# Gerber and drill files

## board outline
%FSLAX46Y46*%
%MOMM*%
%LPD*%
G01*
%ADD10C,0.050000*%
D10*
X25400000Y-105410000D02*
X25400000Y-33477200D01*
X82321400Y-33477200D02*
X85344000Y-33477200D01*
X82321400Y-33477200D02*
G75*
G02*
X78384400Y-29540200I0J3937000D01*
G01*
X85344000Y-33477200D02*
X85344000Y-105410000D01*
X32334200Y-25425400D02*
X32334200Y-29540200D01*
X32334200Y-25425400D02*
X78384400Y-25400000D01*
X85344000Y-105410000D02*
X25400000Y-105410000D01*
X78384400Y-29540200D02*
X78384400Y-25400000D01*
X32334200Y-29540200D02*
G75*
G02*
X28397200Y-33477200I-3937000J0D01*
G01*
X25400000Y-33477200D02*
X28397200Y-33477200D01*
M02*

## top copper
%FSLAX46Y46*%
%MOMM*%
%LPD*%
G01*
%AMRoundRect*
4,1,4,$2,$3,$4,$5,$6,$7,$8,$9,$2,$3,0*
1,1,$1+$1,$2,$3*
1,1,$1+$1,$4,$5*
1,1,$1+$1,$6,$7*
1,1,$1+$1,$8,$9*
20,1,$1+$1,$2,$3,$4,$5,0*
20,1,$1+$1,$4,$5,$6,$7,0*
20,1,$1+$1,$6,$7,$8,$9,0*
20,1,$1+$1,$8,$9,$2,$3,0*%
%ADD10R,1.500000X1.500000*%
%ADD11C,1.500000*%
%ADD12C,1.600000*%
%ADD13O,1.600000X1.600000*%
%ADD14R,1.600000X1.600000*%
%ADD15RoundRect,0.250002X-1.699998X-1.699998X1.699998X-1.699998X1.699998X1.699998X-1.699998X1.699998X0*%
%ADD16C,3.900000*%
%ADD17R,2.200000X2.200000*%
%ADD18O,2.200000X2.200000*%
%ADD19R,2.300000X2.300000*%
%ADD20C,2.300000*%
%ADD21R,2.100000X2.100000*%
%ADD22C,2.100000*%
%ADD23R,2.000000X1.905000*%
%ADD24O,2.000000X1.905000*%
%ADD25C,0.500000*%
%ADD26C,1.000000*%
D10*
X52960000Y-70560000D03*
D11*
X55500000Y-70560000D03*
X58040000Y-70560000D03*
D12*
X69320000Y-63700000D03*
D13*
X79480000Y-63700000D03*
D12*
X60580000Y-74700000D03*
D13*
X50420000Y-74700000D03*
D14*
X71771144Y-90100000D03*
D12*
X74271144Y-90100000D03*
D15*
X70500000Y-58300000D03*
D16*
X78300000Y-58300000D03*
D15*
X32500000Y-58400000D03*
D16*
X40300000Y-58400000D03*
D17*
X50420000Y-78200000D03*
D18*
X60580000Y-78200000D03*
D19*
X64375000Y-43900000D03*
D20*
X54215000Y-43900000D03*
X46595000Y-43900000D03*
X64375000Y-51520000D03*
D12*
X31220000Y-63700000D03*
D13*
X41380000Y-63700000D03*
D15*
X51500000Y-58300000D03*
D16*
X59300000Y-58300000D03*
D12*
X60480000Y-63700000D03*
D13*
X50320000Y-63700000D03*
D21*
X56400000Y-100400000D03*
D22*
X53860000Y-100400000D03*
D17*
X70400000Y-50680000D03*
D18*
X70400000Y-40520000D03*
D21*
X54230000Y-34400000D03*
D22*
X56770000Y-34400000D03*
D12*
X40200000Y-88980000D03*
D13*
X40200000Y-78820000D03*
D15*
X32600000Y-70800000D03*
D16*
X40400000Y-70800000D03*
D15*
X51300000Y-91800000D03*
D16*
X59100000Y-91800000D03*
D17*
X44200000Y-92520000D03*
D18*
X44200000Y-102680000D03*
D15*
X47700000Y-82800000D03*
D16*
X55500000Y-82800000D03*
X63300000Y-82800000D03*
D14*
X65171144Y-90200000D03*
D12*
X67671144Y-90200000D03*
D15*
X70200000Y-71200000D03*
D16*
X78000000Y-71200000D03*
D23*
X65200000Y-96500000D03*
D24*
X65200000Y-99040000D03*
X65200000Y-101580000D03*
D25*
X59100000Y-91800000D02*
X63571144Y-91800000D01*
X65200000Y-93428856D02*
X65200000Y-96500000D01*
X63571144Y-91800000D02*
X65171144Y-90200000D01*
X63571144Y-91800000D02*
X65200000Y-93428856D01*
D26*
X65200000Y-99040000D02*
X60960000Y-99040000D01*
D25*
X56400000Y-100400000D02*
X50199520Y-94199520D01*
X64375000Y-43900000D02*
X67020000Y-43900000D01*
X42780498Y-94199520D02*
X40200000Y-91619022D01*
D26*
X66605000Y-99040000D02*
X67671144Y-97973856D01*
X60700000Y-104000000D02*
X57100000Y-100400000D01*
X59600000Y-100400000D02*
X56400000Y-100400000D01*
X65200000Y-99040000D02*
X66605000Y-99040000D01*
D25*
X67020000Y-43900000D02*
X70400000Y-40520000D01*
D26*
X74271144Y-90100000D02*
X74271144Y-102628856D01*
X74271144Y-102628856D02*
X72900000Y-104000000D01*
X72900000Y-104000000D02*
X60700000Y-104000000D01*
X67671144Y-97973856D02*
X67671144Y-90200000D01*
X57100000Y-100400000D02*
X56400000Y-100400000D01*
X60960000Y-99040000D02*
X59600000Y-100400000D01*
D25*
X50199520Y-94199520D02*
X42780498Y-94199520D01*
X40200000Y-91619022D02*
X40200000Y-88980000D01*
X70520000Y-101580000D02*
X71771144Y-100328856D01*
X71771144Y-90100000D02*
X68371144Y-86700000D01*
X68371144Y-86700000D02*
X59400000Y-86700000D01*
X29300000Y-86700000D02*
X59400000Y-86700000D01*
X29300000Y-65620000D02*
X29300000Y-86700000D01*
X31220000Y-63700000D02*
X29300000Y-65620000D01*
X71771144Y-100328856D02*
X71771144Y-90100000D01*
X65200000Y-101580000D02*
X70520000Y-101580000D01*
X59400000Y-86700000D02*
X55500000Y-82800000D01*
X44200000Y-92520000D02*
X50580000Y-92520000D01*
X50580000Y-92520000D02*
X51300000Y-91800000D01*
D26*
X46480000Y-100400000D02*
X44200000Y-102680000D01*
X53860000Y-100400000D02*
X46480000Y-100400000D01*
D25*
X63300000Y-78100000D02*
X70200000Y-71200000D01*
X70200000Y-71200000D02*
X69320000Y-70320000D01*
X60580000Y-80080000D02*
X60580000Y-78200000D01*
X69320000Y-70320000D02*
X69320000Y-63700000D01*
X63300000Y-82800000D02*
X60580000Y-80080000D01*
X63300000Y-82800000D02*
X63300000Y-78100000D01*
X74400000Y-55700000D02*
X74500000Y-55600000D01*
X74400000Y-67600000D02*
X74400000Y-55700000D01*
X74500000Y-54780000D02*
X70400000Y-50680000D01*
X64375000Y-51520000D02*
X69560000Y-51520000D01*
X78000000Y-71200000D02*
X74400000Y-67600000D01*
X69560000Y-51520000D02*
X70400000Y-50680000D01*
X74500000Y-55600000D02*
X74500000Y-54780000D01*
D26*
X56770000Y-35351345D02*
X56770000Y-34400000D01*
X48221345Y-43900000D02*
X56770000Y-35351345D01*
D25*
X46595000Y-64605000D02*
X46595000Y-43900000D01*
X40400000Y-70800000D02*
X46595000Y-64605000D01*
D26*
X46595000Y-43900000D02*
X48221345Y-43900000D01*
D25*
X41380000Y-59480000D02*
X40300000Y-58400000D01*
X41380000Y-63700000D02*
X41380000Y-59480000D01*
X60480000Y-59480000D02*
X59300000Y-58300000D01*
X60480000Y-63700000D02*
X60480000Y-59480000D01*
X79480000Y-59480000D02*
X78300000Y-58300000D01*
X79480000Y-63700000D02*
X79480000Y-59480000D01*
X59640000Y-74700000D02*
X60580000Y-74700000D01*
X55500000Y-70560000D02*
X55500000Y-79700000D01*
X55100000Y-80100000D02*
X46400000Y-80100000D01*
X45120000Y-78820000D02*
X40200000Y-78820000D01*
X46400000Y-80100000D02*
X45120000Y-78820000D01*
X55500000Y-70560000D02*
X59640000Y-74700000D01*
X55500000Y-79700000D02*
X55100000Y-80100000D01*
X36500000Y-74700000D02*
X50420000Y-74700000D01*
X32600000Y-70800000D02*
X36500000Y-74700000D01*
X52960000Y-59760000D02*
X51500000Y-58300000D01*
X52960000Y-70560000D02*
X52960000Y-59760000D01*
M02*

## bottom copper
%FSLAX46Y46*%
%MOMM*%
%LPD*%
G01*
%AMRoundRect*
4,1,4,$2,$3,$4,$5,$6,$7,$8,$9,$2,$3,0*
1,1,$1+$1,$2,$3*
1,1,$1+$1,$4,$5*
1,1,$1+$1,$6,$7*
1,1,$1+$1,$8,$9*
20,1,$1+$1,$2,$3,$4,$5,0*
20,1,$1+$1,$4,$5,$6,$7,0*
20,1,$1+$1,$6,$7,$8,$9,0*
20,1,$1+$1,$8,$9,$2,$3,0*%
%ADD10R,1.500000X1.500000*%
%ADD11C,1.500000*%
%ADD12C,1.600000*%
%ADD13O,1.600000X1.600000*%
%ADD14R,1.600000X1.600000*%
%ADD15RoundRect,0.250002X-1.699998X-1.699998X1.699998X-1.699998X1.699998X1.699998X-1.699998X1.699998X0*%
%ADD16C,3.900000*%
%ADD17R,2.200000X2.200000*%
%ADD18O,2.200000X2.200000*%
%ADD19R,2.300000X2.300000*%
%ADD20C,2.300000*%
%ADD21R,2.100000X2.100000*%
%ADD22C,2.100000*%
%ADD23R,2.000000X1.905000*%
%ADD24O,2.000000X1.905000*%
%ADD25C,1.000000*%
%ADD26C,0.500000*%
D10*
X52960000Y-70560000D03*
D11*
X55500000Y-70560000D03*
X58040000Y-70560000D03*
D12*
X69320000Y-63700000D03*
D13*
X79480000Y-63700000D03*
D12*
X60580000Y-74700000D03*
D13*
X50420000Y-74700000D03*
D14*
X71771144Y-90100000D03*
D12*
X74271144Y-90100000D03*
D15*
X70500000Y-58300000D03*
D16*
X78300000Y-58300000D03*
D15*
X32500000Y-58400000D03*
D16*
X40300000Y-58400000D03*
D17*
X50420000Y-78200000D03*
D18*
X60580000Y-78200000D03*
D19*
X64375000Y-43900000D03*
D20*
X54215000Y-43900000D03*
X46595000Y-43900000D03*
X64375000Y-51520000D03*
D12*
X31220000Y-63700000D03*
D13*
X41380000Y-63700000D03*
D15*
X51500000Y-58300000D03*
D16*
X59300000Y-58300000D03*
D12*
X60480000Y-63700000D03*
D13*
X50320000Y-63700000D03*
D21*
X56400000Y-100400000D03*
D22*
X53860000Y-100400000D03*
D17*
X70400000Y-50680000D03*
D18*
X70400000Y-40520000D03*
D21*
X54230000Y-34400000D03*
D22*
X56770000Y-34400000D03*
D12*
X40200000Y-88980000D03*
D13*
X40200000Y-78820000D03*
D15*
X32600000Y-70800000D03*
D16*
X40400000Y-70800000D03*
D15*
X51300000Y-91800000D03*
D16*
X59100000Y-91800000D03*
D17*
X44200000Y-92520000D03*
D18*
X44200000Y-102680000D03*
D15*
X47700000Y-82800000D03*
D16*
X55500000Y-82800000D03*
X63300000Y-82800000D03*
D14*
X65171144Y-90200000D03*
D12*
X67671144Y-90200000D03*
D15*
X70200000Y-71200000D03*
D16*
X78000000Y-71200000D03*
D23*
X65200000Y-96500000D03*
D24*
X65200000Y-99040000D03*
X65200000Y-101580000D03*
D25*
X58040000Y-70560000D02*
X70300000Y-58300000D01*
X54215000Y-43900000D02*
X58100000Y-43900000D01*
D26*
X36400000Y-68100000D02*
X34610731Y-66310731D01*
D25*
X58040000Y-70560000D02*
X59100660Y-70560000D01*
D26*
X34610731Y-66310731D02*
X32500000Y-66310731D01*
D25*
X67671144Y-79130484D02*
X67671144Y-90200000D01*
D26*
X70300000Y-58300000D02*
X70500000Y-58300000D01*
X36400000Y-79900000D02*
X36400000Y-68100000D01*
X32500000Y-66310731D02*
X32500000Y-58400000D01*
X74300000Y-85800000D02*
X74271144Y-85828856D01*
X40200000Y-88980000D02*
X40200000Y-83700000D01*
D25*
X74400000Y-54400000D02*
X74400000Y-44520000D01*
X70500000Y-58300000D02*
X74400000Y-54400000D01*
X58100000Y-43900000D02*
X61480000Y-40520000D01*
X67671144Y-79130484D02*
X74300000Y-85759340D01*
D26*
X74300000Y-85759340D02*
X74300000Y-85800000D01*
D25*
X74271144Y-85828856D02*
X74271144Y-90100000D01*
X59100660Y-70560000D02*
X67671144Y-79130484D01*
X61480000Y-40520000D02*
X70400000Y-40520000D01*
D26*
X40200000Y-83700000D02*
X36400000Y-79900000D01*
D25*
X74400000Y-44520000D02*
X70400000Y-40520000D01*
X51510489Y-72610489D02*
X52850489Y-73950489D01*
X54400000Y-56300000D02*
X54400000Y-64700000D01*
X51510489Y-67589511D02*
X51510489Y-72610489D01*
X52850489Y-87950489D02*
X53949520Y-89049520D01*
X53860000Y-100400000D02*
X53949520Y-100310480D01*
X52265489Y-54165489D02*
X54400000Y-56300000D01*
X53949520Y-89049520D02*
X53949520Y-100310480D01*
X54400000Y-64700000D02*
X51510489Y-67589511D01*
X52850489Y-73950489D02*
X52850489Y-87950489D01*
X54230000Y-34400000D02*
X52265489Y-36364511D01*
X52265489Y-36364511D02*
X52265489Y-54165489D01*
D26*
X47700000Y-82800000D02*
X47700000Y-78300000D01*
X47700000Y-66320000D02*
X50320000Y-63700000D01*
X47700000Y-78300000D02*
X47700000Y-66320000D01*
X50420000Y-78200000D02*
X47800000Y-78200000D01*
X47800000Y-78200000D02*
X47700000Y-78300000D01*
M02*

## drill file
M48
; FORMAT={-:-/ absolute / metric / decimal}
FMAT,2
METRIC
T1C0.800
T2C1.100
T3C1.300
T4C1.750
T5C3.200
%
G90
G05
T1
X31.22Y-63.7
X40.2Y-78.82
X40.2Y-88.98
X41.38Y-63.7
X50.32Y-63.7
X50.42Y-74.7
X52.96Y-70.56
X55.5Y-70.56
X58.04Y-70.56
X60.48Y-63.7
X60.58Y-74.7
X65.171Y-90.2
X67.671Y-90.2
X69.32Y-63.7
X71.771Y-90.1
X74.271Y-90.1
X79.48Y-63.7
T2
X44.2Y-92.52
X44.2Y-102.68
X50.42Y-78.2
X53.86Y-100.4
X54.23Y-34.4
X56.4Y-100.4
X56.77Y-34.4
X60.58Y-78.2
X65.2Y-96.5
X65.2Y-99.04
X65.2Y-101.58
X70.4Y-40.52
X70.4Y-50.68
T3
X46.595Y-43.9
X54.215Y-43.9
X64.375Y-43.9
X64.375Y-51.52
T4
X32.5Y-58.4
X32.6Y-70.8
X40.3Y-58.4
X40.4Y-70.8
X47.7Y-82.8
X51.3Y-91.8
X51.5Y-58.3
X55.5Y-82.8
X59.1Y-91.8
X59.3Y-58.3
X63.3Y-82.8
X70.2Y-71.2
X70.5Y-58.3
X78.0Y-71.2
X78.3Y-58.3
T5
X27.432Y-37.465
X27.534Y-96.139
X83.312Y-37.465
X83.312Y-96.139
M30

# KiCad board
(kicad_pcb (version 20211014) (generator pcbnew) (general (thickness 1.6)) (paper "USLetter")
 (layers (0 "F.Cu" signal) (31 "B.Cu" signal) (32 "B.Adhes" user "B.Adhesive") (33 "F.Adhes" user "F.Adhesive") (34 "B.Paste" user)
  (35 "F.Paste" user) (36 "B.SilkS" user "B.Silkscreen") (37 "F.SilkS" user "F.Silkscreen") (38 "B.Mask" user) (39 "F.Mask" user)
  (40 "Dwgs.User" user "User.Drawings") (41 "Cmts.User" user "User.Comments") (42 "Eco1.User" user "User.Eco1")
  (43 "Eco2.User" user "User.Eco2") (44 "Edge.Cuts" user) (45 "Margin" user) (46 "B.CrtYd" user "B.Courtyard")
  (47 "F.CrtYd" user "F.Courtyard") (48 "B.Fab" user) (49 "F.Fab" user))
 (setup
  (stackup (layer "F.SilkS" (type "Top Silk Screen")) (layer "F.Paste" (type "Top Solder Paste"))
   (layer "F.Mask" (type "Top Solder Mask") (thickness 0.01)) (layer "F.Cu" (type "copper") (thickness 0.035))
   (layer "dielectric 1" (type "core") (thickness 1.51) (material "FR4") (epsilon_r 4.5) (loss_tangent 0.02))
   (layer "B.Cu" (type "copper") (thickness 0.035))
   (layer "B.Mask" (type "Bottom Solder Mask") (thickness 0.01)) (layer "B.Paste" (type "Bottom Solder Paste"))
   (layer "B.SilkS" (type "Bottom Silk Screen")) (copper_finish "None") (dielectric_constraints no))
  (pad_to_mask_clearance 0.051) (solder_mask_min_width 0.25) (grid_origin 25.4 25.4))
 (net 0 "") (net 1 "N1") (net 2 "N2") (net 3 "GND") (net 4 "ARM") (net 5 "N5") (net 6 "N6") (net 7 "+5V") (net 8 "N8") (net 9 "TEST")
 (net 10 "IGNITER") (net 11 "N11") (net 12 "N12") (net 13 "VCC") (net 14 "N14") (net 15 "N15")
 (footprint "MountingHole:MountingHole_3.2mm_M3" (layer "F.Cu") (at 27.432 37.465)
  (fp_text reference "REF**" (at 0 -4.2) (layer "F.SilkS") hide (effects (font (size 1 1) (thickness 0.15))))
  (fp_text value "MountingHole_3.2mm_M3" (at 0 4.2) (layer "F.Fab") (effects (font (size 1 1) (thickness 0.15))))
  (pad "" np_thru_hole circle locked (at 0 0) (size 3.2 3.2) (drill 3.2) (layers *.Cu *.Mask)))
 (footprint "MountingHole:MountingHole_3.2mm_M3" (layer "F.Cu") (at 83.312 37.465)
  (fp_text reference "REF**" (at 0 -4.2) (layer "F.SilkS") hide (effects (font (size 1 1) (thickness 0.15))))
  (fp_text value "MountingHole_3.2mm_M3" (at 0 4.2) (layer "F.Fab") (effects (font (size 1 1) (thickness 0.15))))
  (pad "" np_thru_hole circle locked (at 0 0) (size 3.2 3.2) (drill 3.2) (layers *.Cu *.Mask)))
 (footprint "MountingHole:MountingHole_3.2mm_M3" (layer "F.Cu") (at 27.5336 96.139)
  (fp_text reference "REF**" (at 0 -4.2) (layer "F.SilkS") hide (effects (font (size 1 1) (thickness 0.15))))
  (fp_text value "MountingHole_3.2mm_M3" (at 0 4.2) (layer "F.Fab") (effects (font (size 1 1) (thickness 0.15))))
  (pad "" np_thru_hole circle locked (at 0 0) (size 3.2 3.2) (drill 3.2) (layers *.Cu *.Mask)))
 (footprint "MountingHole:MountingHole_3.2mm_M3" (layer "F.Cu") (at 83.312 96.139)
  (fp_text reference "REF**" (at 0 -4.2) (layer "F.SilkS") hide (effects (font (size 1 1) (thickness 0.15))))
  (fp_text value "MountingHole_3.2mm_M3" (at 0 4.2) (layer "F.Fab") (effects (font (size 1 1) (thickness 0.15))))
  (pad "" np_thru_hole circle locked (at 0 0) (size 3.2 3.2) (drill 3.2) (layers *.Cu *.Mask)))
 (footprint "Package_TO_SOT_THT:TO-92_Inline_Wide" (layer "F.Cu") (at 52.96 70.56)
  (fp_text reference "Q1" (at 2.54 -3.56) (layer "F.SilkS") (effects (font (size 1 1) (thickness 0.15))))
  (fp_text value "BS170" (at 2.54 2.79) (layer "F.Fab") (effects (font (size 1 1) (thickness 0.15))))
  (pad "1" thru_hole rect (at 0 0) (size 1.5 1.5) (drill 0.8) (layers *.Cu *.Mask) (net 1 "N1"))
  (pad "2" thru_hole circle (at 2.54 0) (size 1.5 1.5) (drill 0.8) (layers *.Cu *.Mask) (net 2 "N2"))
  (pad "3" thru_hole circle (at 5.08 0) (size 1.5 1.5) (drill 0.8) (layers *.Cu *.Mask) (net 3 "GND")))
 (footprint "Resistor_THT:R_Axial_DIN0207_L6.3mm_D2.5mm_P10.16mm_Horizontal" (layer "F.Cu") (at 69.32 63.7)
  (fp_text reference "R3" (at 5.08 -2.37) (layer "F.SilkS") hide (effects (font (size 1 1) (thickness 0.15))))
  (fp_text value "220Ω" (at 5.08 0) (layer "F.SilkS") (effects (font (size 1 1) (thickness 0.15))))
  (pad "1" thru_hole circle (at 0 0) (size 1.6 1.6) (drill 0.8) (layers *.Cu *.Mask) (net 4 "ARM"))
  (pad "2" thru_hole oval (at 10.16 0) (size 1.6 1.6) (drill 0.8) (layers *.Cu *.Mask) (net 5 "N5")))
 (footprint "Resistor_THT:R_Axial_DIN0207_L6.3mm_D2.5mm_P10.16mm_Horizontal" (layer "F.Cu") (at 60.58 74.7 180)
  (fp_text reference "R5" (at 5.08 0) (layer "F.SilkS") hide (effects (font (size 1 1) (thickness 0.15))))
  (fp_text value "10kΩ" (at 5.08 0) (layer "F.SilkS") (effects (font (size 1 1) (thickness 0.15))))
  (pad "1" thru_hole circle (at 0 0 180) (size 1.6 1.6) (drill 0.8) (layers *.Cu *.Mask) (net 2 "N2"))
  (pad "2" thru_hole oval (at 10.16 0 180) (size 1.6 1.6) (drill 0.8) (layers *.Cu *.Mask) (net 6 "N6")))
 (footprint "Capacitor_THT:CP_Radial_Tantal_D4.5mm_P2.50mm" (layer "F.Cu") (at 71.771144 90.1)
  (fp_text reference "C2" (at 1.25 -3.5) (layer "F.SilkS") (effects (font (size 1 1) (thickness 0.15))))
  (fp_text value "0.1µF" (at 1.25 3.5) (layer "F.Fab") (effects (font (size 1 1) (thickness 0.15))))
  (pad "1" thru_hole rect (at 0 0) (size 1.6 1.6) (drill 0.8) (layers *.Cu *.Mask) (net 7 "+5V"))
  (pad "2" thru_hole circle (at 2.5 0) (size 1.6 1.6) (drill 0.8) (layers *.Cu *.Mask) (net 3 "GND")))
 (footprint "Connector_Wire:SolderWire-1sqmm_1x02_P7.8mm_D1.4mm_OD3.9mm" (layer "F.Cu") (at 70.5 58.3)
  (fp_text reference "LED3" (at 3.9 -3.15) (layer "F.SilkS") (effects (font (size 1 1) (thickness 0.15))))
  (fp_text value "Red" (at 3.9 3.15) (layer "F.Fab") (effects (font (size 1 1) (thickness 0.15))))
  (pad "1" thru_hole roundrect (at 0 0) (size 3.9 3.9) (drill 1.75) (layers *.Cu *.Mask) (roundrect_rratio 0.064103) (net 3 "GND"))
  (pad "2" thru_hole circle (at 7.8 0) (size 3.9 3.9) (drill 1.75) (layers *.Cu *.Mask) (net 5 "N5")))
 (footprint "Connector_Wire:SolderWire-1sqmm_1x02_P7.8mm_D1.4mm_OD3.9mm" (layer "F.Cu") (at 32.5 58.4)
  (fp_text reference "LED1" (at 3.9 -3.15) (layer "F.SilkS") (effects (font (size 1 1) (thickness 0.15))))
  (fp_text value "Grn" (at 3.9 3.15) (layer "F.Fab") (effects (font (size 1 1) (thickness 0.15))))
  (pad "1" thru_hole roundrect (at 0 0) (size 3.9 3.9) (drill 1.75) (layers *.Cu *.Mask) (roundrect_rratio 0.064103) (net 3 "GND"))
  (pad "2" thru_hole circle (at 7.8 0) (size 3.9 3.9) (drill 1.75) (layers *.Cu *.Mask) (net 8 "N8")))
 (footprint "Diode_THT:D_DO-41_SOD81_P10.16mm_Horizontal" (layer "F.Cu") (at 50.42 78.2)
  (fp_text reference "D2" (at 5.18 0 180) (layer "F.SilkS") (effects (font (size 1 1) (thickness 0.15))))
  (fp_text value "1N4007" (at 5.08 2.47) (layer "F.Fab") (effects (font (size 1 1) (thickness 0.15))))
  (pad "1" thru_hole rect (at 0 0) (size 2.2 2.2) (drill 1.1) (layers *.Cu *.Mask) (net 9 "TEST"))
  (pad "2" thru_hole oval (at 10.16 0) (size 2.2 2.2) (drill 1.1) (layers *.Cu *.Mask) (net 4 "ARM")))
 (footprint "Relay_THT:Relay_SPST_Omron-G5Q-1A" (layer "F.Cu") (at 64.375 43.9 180)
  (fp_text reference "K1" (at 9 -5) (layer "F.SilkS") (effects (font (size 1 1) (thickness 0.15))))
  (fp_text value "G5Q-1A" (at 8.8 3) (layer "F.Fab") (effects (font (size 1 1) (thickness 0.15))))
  (pad "1" thru_hole rect (at 0 0) (size 2.3 2.3) (drill 1.3) (layers *.Cu *.Mask) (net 3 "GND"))
  (pad "2" thru_hole circle (at 10.16 0) (size 2.3 2.3) (drill 1.3) (layers *.Cu *.Mask) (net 3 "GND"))
  (pad "3" thru_hole circle (at 17.78 0) (size 2.3 2.3) (drill 1.3) (layers *.Cu *.Mask) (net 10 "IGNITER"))
  (pad "5" thru_hole circle (at 0 -7.62) (size 2.3 2.3) (drill 1.3) (layers *.Cu *.Mask) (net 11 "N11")))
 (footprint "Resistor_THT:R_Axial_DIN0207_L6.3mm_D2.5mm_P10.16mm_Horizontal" (layer "F.Cu") (at 31.22 63.7)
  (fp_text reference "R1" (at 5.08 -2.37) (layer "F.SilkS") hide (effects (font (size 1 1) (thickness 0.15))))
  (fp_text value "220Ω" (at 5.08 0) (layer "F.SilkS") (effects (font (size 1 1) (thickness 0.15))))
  (pad "1" thru_hole circle (at 0 0) (size 1.6 1.6) (drill 0.8) (layers *.Cu *.Mask) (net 7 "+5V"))
  (pad "2" thru_hole oval (at 10.16 0) (size 1.6 1.6) (drill 0.8) (layers *.Cu *.Mask) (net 8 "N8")))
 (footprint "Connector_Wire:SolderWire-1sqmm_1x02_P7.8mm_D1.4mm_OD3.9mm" (layer "F.Cu") (at 51.5 58.3)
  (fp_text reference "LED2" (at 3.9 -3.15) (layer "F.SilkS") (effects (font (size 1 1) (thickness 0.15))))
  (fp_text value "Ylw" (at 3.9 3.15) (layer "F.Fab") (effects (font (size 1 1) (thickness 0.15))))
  (pad "1" thru_hole roundrect (at 0 0) (size 3.9 3.9) (drill 1.75) (layers *.Cu *.Mask) (roundrect_rratio 0.064103) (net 1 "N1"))
  (pad "2" thru_hole circle (at 7.8 0) (size 3.9 3.9) (drill 1.75) (layers *.Cu *.Mask) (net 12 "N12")))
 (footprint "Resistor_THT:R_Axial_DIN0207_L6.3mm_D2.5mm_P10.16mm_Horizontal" (layer "F.Cu") (at 60.48 63.7 180)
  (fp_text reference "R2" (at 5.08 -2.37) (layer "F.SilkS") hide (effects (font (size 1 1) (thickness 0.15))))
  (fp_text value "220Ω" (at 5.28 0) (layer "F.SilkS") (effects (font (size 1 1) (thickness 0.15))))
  (pad "1" thru_hole circle (at 0 0 180) (size 1.6 1.6) (drill 0.8) (layers *.Cu *.Mask) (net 12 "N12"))
  (pad "2" thru_hole oval (at 10.16 0 180) (size 1.6 1.6) (drill 0.8) (layers *.Cu *.Mask) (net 9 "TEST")))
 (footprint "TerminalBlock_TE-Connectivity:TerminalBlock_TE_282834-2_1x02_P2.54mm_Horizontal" (layer "F.Cu") (at 56.4 100.4 180)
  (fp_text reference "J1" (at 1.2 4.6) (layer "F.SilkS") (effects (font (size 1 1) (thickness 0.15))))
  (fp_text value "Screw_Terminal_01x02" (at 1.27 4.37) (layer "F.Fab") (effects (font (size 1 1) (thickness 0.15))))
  (pad "1" thru_hole rect (at 0 0 180) (size 2.1 2.1) (drill 1.1) (layers *.Cu *.Mask) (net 3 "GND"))
  (pad "2" thru_hole circle (at 2.54 0 180) (size 2.1 2.1) (drill 1.1) (layers *.Cu *.Mask) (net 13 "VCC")))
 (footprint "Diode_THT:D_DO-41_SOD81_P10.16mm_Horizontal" (layer "F.Cu") (at 70.4 50.68 90)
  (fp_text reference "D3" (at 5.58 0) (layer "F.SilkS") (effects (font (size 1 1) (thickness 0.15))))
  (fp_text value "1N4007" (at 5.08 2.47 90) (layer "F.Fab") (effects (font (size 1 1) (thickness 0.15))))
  (pad "1" thru_hole rect (at 0 0 90) (size 2.2 2.2) (drill 1.1) (layers *.Cu *.Mask) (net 11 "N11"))
  (pad "2" thru_hole oval (at 10.16 0 90) (size 2.2 2.2) (drill 1.1) (layers *.Cu *.Mask) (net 3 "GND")))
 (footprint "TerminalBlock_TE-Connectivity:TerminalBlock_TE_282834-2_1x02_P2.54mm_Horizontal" (layer "F.Cu") (at 54.23 34.4)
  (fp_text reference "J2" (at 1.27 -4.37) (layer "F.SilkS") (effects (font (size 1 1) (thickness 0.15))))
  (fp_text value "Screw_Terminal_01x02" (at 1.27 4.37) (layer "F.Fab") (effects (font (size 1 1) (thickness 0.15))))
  (pad "1" thru_hole rect (at 0 0) (size 2.1 2.1) (drill 1.1) (layers *.Cu *.Mask) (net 13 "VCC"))
  (pad "2" thru_hole circle (at 2.54 0) (size 2.1 2.1) (drill 1.1) (layers *.Cu *.Mask) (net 10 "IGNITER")))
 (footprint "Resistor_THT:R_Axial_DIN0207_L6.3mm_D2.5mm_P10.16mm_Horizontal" (layer "F.Cu") (at 40.2 88.98 90)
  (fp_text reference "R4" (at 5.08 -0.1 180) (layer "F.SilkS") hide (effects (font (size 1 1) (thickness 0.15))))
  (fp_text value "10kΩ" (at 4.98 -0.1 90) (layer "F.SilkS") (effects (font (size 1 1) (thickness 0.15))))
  (pad "1" thru_hole circle (at 0 0 90) (size 1.6 1.6) (drill 0.8) (layers *.Cu *.Mask) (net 3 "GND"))
  (pad "2" thru_hole oval (at 10.16 0 90) (size 1.6 1.6) (drill 0.8) (layers *.Cu *.Mask) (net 2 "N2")))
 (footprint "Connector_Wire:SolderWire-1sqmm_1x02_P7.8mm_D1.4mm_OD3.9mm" (layer "F.Cu") (at 32.6 70.8)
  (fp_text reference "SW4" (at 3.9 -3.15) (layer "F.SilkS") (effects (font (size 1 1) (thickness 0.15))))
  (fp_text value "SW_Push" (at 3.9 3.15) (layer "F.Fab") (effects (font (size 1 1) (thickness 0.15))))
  (pad "1" thru_hole roundrect (at 0 0) (size 3.9 3.9) (drill 1.75) (layers *.Cu *.Mask) (roundrect_rratio 0.064103) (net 6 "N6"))
  (pad "2" thru_hole circle (at 7.8 0) (size 3.9 3.9) (drill 1.75) (layers *.Cu *.Mask) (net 10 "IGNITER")))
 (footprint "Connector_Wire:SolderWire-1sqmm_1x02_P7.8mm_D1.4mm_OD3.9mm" (layer "F.Cu") (at 51.3 91.8)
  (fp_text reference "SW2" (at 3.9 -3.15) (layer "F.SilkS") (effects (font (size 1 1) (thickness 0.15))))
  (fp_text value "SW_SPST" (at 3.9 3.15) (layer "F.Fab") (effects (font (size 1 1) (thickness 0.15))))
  (pad "1" thru_hole roundrect (at 0 0) (size 3.9 3.9) (drill 1.75) (layers *.Cu *.Mask) (roundrect_rratio 0.064103) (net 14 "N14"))
  (pad "2" thru_hole circle (at 7.8 0) (size 3.9 3.9) (drill 1.75) (layers *.Cu *.Mask) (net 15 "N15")))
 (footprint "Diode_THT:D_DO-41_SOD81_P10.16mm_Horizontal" (layer "F.Cu") (at 44.2 92.52 -90)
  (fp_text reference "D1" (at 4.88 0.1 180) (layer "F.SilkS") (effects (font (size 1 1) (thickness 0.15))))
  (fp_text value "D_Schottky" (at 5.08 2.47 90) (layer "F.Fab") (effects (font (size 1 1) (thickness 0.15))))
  (pad "1" thru_hole rect (at 0 0 270) (size 2.2 2.2) (drill 1.1) (layers *.Cu *.Mask) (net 14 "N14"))
  (pad "2" thru_hole oval (at 10.16 0 270) (size 2.2 2.2) (drill 1.1) (layers *.Cu *.Mask) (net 13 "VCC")))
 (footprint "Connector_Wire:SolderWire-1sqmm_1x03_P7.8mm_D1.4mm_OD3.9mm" (layer "F.Cu") (at 47.7 82.8)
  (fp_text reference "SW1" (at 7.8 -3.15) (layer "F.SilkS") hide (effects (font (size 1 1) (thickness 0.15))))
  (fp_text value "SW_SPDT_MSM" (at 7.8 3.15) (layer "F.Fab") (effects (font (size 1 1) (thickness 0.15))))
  (pad "1" thru_hole roundrect (at 0 0) (size 3.9 3.9) (drill 1.75) (layers *.Cu *.Mask) (roundrect_rratio 0.064103) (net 9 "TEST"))
  (pad "2" thru_hole circle (at 7.8 0) (size 3.9 3.9) (drill 1.75) (layers *.Cu *.Mask) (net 7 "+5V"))
  (pad "3" thru_hole circle (at 15.6 0) (size 3.9 3.9) (drill 1.75) (layers *.Cu *.Mask) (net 4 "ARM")))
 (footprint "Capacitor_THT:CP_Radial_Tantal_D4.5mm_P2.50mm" (layer "F.Cu") (at 65.171144 90.2)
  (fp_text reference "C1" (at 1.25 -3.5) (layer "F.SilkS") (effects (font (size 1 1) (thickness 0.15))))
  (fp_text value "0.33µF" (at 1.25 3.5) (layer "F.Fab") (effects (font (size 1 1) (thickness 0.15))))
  (pad "1" thru_hole rect (at 0 0) (size 1.6 1.6) (drill 0.8) (layers *.Cu *.Mask) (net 15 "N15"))
  (pad "2" thru_hole circle (at 2.5 0) (size 1.6 1.6) (drill 0.8) (layers *.Cu *.Mask) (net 3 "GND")))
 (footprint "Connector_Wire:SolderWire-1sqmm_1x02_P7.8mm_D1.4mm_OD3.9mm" (layer "F.Cu") (at 70.2 71.2)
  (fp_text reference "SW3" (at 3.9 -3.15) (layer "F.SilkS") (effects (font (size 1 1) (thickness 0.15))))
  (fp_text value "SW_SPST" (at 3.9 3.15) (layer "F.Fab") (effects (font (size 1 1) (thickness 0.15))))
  (pad "1" thru_hole roundrect (at 0 0) (size 3.9 3.9) (drill 1.75) (layers *.Cu *.Mask) (roundrect_rratio 0.064103) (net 4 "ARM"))
  (pad "2" thru_hole circle (at 7.8 0) (size 3.9 3.9) (drill 1.75) (layers *.Cu *.Mask) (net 11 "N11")))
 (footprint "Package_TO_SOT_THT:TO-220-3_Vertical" (layer "F.Cu") (at 65.2 96.5 -90)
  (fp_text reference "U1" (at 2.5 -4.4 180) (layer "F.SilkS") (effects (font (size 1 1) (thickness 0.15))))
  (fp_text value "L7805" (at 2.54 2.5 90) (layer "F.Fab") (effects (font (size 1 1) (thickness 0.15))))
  (pad "1" thru_hole rect (at 0 0 270) (size 1.905 2) (drill 1.1) (layers *.Cu *.Mask) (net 15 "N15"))
  (pad "2" thru_hole oval (at 2.54 0 270) (size 1.905 2) (drill 1.1) (layers *.Cu *.Mask) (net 3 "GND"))
  (pad "3" thru_hole oval (at 5.08 0 270) (size 1.905 2) (drill 1.1) (layers *.Cu *.Mask) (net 7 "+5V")))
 (gr_line (start 25.4 105.41) (end 25.4 33.4772) (layer "Edge.Cuts") (width 0.05))
 (gr_line (start 82.3214 33.4772) (end 85.344 33.4772) (layer "Edge.Cuts") (width 0.05))
 (gr_arc (start 82.3214 33.4772) (mid 79.537521 32.324079) (end 78.3844 29.5402) (layer "Edge.Cuts") (width 0.05))
 (gr_line (start 85.344 33.4772) (end 85.344 105.41) (layer "Edge.Cuts") (width 0.05))
 (gr_line (start 32.3342 25.4254) (end 32.3342 29.5402) (layer "Edge.Cuts") (width 0.05))
 (gr_line (start 32.3342 25.4254) (end 78.3844 25.4) (layer "Edge.Cuts") (width 0.05))
 (gr_line (start 85.344 105.41) (end 25.4 105.41) (layer "Edge.Cuts") (width 0.05))
 (gr_line (start 78.3844 29.5402) (end 78.3844 25.4) (layer "Edge.Cuts") (width 0.05))
 (gr_arc (start 32.3342 29.5402) (mid 31.181079 32.324079) (end 28.3972 33.4772) (layer "Edge.Cuts") (width 0.05))
 (gr_line (start 25.4 33.4772) (end 28.3972 33.4772) (layer "Edge.Cuts") (width 0.05))
 (segment (start 59.1 91.8) (end 63.571144 91.8) (width 0.5) (layer "F.Cu") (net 15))
 (segment (start 65.2 93.428856) (end 65.2 96.5) (width 0.5) (layer "F.Cu") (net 15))
 (segment (start 63.571144 91.8) (end 65.171144 90.2) (width 0.5) (layer "F.Cu") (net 15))
 (segment (start 63.571144 91.8) (end 65.2 93.428856) (width 0.5) (layer "F.Cu") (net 15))
 (segment (start 65.2 99.04) (end 60.96 99.04) (width 1) (layer "F.Cu") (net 3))
 (segment (start 56.4 100.4) (end 50.19952 94.19952) (width 0.5) (layer "F.Cu") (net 3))
 (segment (start 64.375 43.9) (end 67.02 43.9) (width 0.5) (layer "F.Cu") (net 3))
 (segment (start 42.780498 94.19952) (end 40.2 91.619022) (width 0.5) (layer "F.Cu") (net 3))
 (segment (start 66.605 99.04) (end 67.671144 97.973856) (width 1) (layer "F.Cu") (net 3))
 (segment (start 60.7 104) (end 57.1 100.4) (width 1) (layer "F.Cu") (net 3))
 (segment (start 59.6 100.4) (end 56.4 100.4) (width 1) (layer "F.Cu") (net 3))
 (segment (start 65.2 99.04) (end 66.605 99.04) (width 1) (layer "F.Cu") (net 3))
 (segment (start 67.02 43.9) (end 70.4 40.52) (width 0.5) (layer "F.Cu") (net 3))
 (segment (start 74.271144 90.1) (end 74.271144 102.628856) (width 1) (layer "F.Cu") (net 3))
 (segment (start 74.271144 102.628856) (end 72.9 104) (width 1) (layer "F.Cu") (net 3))
 (segment (start 72.9 104) (end 60.7 104) (width 1) (layer "F.Cu") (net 3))
 (segment (start 67.671144 97.973856) (end 67.671144 90.2) (width 1) (layer "F.Cu") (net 3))
 (segment (start 57.1 100.4) (end 56.4 100.4) (width 1) (layer "F.Cu") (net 3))
 (segment (start 60.96 99.04) (end 59.6 100.4) (width 1) (layer "F.Cu") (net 3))
 (segment (start 50.19952 94.19952) (end 42.780498 94.19952) (width 0.5) (layer "F.Cu") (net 3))
 (segment (start 40.2 91.619022) (end 40.2 88.98) (width 0.5) (layer "F.Cu") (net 3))
 (segment (start 58.04 70.56) (end 70.3 58.3) (width 1) (layer "B.Cu") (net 3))
 (segment (start 54.215 43.9) (end 58.1 43.9) (width 1) (layer "B.Cu") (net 3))
 (segment (start 36.4 68.1) (end 34.610731 66.310731) (width 0.5) (layer "B.Cu") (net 3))
 (segment (start 58.04 70.56) (end 59.10066 70.56) (width 1) (layer "B.Cu") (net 3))
 (segment (start 34.610731 66.310731) (end 32.5 66.310731) (width 0.5) (layer "B.Cu") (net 3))
 (segment (start 67.671144 79.130484) (end 67.671144 90.2) (width 1) (layer "B.Cu") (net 3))
 (segment (start 70.3 58.3) (end 70.5 58.3) (width 0.5) (layer "B.Cu") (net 3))
 (segment (start 36.4 79.9) (end 36.4 68.1) (width 0.5) (layer "B.Cu") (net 3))
 (segment (start 32.5 66.310731) (end 32.5 58.4) (width 0.5) (layer "B.Cu") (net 3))
 (segment (start 74.3 85.8) (end 74.271144 85.828856) (width 0.5) (layer "B.Cu") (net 3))
 (segment (start 40.2 88.98) (end 40.2 83.7) (width 0.5) (layer "B.Cu") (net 3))
 (segment (start 74.4 54.4) (end 74.4 44.52) (width 1) (layer "B.Cu") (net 3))
 (segment (start 70.5 58.3) (end 74.4 54.4) (width 1) (layer "B.Cu") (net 3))
 (segment (start 58.1 43.9) (end 61.48 40.52) (width 1) (layer "B.Cu") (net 3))
 (segment (start 67.671144 79.130484) (end 74.3 85.75934) (width 1) (layer "B.Cu") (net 3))
 (segment (start 74.3 85.75934) (end 74.3 85.8) (width 0.5) (layer "B.Cu") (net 3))
 (segment (start 74.271144 85.828856) (end 74.271144 90.1) (width 1) (layer "B.Cu") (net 3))
 (segment (start 59.10066 70.56) (end 67.671144 79.130484) (width 1) (layer "B.Cu") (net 3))
 (segment (start 61.48 40.52) (end 70.4 40.52) (width 1) (layer "B.Cu") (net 3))
 (segment (start 40.2 83.7) (end 36.4 79.9) (width 0.5) (layer "B.Cu") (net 3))
 (segment (start 74.4 44.52) (end 70.4 40.52) (width 1) (layer "B.Cu") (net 3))
 (segment (start 70.52 101.58) (end 71.771144 100.328856) (width 0.5) (layer "F.Cu") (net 7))
 (segment (start 71.771144 90.1) (end 68.371144 86.7) (width 0.5) (layer "F.Cu") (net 7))
 (segment (start 68.371144 86.7) (end 59.4 86.7) (width 0.5) (layer "F.Cu") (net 7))
 (segment (start 29.3 86.7) (end 59.4 86.7) (width 0.5) (layer "F.Cu") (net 7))
 (segment (start 29.3 65.62) (end 29.3 86.7) (width 0.5) (layer "F.Cu") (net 7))
 (segment (start 31.22 63.7) (end 29.3 65.62) (width 0.5) (layer "F.Cu") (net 7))
 (segment (start 71.771144 100.328856) (end 71.771144 90.1) (width 0.5) (layer "F.Cu") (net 7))
 (segment (start 65.2 101.58) (end 70.52 101.58) (width 0.5) (layer "F.Cu") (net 7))
 (segment (start 59.4 86.7) (end 55.5 82.8) (width 0.5) (layer "F.Cu") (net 7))
 (segment (start 44.2 92.52) (end 50.58 92.52) (width 0.5) (layer "F.Cu") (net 14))
 (segment (start 50.58 92.52) (end 51.3 91.8) (width 0.5) (layer "F.Cu") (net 14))
 (segment (start 46.48 100.4) (end 44.2 102.68) (width 1) (layer "F.Cu") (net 13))
 (segment (start 53.86 100.4) (end 46.48 100.4) (width 1) (layer "F.Cu") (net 13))
 (segment (start 51.510489 72.610489) (end 52.850489 73.950489) (width 1) (layer "B.Cu") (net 13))
 (segment (start 54.4 56.3) (end 54.4 64.7) (width 1) (layer "B.Cu") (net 13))
 (segment (start 51.510489 67.589511) (end 51.510489 72.610489) (width 1) (layer "B.Cu") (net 13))
 (segment (start 52.850489 87.950489) (end 53.94952 89.04952) (width 1) (layer "B.Cu") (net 13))
 (segment (start 53.86 100.4) (end 53.94952 100.31048) (width 1) (layer "B.Cu") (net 13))
 (segment (start 52.265489 54.165489) (end 54.4 56.3) (width 1) (layer "B.Cu") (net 13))
 (segment (start 53.94952 89.04952) (end 53.94952 100.31048) (width 1) (layer "B.Cu") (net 13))
 (segment (start 54.4 64.7) (end 51.510489 67.589511) (width 1) (layer "B.Cu") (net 13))
 (segment (start 52.850489 73.950489) (end 52.850489 87.950489) (width 1) (layer "B.Cu") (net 13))
 (segment (start 54.23 34.4) (end 52.265489 36.364511) (width 1) (layer "B.Cu") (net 13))
 (segment (start 52.265489 36.364511) (end 52.265489 54.165489) (width 1) (layer "B.Cu") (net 13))
 (segment (start 47.7 82.8) (end 47.7 78.3) (width 0.5) (layer "B.Cu") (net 9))
 (segment (start 47.7 66.32) (end 50.32 63.7) (width 0.5) (layer "B.Cu") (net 9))
 (segment (start 47.7 78.3) (end 47.7 66.32) (width 0.5) (layer "B.Cu") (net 9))
 (segment (start 50.42 78.2) (end 47.8 78.2) (width 0.5) (layer "B.Cu") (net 9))
 (segment (start 47.8 78.2) (end 47.7 78.3) (width 0.5) (layer "B.Cu") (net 9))
 (segment (start 63.3 78.1) (end 70.2 71.2) (width 0.5) (layer "F.Cu") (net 4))
 (segment (start 70.2 71.2) (end 69.32 70.32) (width 0.5) (layer "F.Cu") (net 4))
 (segment (start 60.58 80.08) (end 60.58 78.2) (width 0.5) (layer "F.Cu") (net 4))
 (segment (start 69.32 70.32) (end 69.32 63.7) (width 0.5) (layer "F.Cu") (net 4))
 (segment (start 63.3 82.8) (end 60.58 80.08) (width 0.5) (layer "F.Cu") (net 4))
 (segment (start 63.3 82.8) (end 63.3 78.1) (width 0.5) (layer "F.Cu") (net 4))
 (segment (start 74.4 55.7) (end 74.5 55.6) (width 0.5) (layer "F.Cu") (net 11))
 (segment (start 74.4 67.6) (end 74.4 55.7) (width 0.5) (layer "F.Cu") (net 11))
 (segment (start 74.5 54.78) (end 70.4 50.68) (width 0.5) (layer "F.Cu") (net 11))
 (segment (start 64.375 51.52) (end 69.56 51.52) (width 0.5) (layer "F.Cu") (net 11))
 (segment (start 78 71.2) (end 74.4 67.6) (width 0.5) (layer "F.Cu") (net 11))
 (segment (start 69.56 51.52) (end 70.4 50.68) (width 0.5) (layer "F.Cu") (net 11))
 (segment (start 74.5 55.6) (end 74.5 54.78) (width 0.5) (layer "F.Cu") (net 11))
 (segment (start 56.77 35.351345) (end 56.77 34.4) (width 1) (layer "F.Cu") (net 10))
 (segment (start 48.221345 43.9) (end 56.77 35.351345) (width 1) (layer "F.Cu") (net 10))
 (segment (start 46.595 64.605) (end 46.595 43.9) (width 0.5) (layer "F.Cu") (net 10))
 (segment (start 40.4 70.8) (end 46.595 64.605) (width 0.5) (layer "F.Cu") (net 10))
 (segment (start 46.595 43.9) (end 48.221345 43.9) (width 1) (layer "F.Cu") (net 10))
 (segment (start 41.38 59.48) (end 40.3 58.4) (width 0.5) (layer "F.Cu") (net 8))
 (segment (start 41.38 63.7) (end 41.38 59.48) (width 0.5) (layer "F.Cu") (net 8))
 (segment (start 60.48 59.48) (end 59.3 58.3) (width 0.5) (layer "F.Cu") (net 12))
 (segment (start 60.48 63.7) (end 60.48 59.48) (width 0.5) (layer "F.Cu") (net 12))
 (segment (start 79.48 59.48) (end 78.3 58.3) (width 0.5) (layer "F.Cu") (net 5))
 (segment (start 79.48 63.7) (end 79.48 59.48) (width 0.5) (layer "F.Cu") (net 5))
 (segment (start 59.64 74.7) (end 60.58 74.7) (width 0.5) (layer "F.Cu") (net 2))
 (segment (start 55.5 70.56) (end 55.5 79.7) (width 0.5) (layer "F.Cu") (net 2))
 (segment (start 55.1 80.1) (end 46.4 80.1) (width 0.5) (layer "F.Cu") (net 2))
 (segment (start 45.12 78.82) (end 40.2 78.82) (width 0.5) (layer "F.Cu") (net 2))
 (segment (start 46.4 80.1) (end 45.12 78.82) (width 0.5) (layer "F.Cu") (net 2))
 (segment (start 55.5 70.56) (end 59.64 74.7) (width 0.5) (layer "F.Cu") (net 2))
 (segment (start 55.5 79.7) (end 55.1 80.1) (width 0.5) (layer "F.Cu") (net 2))
 (segment (start 36.5 74.7) (end 50.42 74.7) (width 0.5) (layer "F.Cu") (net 6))
 (segment (start 32.6 70.8) (end 36.5 74.7) (width 0.5) (layer "F.Cu") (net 6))
 (segment (start 52.96 59.76) (end 51.5 58.3) (width 0.5) (layer "F.Cu") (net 1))
 (segment (start 52.96 70.56) (end 52.96 59.76) (width 0.5) (layer "F.Cu") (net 1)))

